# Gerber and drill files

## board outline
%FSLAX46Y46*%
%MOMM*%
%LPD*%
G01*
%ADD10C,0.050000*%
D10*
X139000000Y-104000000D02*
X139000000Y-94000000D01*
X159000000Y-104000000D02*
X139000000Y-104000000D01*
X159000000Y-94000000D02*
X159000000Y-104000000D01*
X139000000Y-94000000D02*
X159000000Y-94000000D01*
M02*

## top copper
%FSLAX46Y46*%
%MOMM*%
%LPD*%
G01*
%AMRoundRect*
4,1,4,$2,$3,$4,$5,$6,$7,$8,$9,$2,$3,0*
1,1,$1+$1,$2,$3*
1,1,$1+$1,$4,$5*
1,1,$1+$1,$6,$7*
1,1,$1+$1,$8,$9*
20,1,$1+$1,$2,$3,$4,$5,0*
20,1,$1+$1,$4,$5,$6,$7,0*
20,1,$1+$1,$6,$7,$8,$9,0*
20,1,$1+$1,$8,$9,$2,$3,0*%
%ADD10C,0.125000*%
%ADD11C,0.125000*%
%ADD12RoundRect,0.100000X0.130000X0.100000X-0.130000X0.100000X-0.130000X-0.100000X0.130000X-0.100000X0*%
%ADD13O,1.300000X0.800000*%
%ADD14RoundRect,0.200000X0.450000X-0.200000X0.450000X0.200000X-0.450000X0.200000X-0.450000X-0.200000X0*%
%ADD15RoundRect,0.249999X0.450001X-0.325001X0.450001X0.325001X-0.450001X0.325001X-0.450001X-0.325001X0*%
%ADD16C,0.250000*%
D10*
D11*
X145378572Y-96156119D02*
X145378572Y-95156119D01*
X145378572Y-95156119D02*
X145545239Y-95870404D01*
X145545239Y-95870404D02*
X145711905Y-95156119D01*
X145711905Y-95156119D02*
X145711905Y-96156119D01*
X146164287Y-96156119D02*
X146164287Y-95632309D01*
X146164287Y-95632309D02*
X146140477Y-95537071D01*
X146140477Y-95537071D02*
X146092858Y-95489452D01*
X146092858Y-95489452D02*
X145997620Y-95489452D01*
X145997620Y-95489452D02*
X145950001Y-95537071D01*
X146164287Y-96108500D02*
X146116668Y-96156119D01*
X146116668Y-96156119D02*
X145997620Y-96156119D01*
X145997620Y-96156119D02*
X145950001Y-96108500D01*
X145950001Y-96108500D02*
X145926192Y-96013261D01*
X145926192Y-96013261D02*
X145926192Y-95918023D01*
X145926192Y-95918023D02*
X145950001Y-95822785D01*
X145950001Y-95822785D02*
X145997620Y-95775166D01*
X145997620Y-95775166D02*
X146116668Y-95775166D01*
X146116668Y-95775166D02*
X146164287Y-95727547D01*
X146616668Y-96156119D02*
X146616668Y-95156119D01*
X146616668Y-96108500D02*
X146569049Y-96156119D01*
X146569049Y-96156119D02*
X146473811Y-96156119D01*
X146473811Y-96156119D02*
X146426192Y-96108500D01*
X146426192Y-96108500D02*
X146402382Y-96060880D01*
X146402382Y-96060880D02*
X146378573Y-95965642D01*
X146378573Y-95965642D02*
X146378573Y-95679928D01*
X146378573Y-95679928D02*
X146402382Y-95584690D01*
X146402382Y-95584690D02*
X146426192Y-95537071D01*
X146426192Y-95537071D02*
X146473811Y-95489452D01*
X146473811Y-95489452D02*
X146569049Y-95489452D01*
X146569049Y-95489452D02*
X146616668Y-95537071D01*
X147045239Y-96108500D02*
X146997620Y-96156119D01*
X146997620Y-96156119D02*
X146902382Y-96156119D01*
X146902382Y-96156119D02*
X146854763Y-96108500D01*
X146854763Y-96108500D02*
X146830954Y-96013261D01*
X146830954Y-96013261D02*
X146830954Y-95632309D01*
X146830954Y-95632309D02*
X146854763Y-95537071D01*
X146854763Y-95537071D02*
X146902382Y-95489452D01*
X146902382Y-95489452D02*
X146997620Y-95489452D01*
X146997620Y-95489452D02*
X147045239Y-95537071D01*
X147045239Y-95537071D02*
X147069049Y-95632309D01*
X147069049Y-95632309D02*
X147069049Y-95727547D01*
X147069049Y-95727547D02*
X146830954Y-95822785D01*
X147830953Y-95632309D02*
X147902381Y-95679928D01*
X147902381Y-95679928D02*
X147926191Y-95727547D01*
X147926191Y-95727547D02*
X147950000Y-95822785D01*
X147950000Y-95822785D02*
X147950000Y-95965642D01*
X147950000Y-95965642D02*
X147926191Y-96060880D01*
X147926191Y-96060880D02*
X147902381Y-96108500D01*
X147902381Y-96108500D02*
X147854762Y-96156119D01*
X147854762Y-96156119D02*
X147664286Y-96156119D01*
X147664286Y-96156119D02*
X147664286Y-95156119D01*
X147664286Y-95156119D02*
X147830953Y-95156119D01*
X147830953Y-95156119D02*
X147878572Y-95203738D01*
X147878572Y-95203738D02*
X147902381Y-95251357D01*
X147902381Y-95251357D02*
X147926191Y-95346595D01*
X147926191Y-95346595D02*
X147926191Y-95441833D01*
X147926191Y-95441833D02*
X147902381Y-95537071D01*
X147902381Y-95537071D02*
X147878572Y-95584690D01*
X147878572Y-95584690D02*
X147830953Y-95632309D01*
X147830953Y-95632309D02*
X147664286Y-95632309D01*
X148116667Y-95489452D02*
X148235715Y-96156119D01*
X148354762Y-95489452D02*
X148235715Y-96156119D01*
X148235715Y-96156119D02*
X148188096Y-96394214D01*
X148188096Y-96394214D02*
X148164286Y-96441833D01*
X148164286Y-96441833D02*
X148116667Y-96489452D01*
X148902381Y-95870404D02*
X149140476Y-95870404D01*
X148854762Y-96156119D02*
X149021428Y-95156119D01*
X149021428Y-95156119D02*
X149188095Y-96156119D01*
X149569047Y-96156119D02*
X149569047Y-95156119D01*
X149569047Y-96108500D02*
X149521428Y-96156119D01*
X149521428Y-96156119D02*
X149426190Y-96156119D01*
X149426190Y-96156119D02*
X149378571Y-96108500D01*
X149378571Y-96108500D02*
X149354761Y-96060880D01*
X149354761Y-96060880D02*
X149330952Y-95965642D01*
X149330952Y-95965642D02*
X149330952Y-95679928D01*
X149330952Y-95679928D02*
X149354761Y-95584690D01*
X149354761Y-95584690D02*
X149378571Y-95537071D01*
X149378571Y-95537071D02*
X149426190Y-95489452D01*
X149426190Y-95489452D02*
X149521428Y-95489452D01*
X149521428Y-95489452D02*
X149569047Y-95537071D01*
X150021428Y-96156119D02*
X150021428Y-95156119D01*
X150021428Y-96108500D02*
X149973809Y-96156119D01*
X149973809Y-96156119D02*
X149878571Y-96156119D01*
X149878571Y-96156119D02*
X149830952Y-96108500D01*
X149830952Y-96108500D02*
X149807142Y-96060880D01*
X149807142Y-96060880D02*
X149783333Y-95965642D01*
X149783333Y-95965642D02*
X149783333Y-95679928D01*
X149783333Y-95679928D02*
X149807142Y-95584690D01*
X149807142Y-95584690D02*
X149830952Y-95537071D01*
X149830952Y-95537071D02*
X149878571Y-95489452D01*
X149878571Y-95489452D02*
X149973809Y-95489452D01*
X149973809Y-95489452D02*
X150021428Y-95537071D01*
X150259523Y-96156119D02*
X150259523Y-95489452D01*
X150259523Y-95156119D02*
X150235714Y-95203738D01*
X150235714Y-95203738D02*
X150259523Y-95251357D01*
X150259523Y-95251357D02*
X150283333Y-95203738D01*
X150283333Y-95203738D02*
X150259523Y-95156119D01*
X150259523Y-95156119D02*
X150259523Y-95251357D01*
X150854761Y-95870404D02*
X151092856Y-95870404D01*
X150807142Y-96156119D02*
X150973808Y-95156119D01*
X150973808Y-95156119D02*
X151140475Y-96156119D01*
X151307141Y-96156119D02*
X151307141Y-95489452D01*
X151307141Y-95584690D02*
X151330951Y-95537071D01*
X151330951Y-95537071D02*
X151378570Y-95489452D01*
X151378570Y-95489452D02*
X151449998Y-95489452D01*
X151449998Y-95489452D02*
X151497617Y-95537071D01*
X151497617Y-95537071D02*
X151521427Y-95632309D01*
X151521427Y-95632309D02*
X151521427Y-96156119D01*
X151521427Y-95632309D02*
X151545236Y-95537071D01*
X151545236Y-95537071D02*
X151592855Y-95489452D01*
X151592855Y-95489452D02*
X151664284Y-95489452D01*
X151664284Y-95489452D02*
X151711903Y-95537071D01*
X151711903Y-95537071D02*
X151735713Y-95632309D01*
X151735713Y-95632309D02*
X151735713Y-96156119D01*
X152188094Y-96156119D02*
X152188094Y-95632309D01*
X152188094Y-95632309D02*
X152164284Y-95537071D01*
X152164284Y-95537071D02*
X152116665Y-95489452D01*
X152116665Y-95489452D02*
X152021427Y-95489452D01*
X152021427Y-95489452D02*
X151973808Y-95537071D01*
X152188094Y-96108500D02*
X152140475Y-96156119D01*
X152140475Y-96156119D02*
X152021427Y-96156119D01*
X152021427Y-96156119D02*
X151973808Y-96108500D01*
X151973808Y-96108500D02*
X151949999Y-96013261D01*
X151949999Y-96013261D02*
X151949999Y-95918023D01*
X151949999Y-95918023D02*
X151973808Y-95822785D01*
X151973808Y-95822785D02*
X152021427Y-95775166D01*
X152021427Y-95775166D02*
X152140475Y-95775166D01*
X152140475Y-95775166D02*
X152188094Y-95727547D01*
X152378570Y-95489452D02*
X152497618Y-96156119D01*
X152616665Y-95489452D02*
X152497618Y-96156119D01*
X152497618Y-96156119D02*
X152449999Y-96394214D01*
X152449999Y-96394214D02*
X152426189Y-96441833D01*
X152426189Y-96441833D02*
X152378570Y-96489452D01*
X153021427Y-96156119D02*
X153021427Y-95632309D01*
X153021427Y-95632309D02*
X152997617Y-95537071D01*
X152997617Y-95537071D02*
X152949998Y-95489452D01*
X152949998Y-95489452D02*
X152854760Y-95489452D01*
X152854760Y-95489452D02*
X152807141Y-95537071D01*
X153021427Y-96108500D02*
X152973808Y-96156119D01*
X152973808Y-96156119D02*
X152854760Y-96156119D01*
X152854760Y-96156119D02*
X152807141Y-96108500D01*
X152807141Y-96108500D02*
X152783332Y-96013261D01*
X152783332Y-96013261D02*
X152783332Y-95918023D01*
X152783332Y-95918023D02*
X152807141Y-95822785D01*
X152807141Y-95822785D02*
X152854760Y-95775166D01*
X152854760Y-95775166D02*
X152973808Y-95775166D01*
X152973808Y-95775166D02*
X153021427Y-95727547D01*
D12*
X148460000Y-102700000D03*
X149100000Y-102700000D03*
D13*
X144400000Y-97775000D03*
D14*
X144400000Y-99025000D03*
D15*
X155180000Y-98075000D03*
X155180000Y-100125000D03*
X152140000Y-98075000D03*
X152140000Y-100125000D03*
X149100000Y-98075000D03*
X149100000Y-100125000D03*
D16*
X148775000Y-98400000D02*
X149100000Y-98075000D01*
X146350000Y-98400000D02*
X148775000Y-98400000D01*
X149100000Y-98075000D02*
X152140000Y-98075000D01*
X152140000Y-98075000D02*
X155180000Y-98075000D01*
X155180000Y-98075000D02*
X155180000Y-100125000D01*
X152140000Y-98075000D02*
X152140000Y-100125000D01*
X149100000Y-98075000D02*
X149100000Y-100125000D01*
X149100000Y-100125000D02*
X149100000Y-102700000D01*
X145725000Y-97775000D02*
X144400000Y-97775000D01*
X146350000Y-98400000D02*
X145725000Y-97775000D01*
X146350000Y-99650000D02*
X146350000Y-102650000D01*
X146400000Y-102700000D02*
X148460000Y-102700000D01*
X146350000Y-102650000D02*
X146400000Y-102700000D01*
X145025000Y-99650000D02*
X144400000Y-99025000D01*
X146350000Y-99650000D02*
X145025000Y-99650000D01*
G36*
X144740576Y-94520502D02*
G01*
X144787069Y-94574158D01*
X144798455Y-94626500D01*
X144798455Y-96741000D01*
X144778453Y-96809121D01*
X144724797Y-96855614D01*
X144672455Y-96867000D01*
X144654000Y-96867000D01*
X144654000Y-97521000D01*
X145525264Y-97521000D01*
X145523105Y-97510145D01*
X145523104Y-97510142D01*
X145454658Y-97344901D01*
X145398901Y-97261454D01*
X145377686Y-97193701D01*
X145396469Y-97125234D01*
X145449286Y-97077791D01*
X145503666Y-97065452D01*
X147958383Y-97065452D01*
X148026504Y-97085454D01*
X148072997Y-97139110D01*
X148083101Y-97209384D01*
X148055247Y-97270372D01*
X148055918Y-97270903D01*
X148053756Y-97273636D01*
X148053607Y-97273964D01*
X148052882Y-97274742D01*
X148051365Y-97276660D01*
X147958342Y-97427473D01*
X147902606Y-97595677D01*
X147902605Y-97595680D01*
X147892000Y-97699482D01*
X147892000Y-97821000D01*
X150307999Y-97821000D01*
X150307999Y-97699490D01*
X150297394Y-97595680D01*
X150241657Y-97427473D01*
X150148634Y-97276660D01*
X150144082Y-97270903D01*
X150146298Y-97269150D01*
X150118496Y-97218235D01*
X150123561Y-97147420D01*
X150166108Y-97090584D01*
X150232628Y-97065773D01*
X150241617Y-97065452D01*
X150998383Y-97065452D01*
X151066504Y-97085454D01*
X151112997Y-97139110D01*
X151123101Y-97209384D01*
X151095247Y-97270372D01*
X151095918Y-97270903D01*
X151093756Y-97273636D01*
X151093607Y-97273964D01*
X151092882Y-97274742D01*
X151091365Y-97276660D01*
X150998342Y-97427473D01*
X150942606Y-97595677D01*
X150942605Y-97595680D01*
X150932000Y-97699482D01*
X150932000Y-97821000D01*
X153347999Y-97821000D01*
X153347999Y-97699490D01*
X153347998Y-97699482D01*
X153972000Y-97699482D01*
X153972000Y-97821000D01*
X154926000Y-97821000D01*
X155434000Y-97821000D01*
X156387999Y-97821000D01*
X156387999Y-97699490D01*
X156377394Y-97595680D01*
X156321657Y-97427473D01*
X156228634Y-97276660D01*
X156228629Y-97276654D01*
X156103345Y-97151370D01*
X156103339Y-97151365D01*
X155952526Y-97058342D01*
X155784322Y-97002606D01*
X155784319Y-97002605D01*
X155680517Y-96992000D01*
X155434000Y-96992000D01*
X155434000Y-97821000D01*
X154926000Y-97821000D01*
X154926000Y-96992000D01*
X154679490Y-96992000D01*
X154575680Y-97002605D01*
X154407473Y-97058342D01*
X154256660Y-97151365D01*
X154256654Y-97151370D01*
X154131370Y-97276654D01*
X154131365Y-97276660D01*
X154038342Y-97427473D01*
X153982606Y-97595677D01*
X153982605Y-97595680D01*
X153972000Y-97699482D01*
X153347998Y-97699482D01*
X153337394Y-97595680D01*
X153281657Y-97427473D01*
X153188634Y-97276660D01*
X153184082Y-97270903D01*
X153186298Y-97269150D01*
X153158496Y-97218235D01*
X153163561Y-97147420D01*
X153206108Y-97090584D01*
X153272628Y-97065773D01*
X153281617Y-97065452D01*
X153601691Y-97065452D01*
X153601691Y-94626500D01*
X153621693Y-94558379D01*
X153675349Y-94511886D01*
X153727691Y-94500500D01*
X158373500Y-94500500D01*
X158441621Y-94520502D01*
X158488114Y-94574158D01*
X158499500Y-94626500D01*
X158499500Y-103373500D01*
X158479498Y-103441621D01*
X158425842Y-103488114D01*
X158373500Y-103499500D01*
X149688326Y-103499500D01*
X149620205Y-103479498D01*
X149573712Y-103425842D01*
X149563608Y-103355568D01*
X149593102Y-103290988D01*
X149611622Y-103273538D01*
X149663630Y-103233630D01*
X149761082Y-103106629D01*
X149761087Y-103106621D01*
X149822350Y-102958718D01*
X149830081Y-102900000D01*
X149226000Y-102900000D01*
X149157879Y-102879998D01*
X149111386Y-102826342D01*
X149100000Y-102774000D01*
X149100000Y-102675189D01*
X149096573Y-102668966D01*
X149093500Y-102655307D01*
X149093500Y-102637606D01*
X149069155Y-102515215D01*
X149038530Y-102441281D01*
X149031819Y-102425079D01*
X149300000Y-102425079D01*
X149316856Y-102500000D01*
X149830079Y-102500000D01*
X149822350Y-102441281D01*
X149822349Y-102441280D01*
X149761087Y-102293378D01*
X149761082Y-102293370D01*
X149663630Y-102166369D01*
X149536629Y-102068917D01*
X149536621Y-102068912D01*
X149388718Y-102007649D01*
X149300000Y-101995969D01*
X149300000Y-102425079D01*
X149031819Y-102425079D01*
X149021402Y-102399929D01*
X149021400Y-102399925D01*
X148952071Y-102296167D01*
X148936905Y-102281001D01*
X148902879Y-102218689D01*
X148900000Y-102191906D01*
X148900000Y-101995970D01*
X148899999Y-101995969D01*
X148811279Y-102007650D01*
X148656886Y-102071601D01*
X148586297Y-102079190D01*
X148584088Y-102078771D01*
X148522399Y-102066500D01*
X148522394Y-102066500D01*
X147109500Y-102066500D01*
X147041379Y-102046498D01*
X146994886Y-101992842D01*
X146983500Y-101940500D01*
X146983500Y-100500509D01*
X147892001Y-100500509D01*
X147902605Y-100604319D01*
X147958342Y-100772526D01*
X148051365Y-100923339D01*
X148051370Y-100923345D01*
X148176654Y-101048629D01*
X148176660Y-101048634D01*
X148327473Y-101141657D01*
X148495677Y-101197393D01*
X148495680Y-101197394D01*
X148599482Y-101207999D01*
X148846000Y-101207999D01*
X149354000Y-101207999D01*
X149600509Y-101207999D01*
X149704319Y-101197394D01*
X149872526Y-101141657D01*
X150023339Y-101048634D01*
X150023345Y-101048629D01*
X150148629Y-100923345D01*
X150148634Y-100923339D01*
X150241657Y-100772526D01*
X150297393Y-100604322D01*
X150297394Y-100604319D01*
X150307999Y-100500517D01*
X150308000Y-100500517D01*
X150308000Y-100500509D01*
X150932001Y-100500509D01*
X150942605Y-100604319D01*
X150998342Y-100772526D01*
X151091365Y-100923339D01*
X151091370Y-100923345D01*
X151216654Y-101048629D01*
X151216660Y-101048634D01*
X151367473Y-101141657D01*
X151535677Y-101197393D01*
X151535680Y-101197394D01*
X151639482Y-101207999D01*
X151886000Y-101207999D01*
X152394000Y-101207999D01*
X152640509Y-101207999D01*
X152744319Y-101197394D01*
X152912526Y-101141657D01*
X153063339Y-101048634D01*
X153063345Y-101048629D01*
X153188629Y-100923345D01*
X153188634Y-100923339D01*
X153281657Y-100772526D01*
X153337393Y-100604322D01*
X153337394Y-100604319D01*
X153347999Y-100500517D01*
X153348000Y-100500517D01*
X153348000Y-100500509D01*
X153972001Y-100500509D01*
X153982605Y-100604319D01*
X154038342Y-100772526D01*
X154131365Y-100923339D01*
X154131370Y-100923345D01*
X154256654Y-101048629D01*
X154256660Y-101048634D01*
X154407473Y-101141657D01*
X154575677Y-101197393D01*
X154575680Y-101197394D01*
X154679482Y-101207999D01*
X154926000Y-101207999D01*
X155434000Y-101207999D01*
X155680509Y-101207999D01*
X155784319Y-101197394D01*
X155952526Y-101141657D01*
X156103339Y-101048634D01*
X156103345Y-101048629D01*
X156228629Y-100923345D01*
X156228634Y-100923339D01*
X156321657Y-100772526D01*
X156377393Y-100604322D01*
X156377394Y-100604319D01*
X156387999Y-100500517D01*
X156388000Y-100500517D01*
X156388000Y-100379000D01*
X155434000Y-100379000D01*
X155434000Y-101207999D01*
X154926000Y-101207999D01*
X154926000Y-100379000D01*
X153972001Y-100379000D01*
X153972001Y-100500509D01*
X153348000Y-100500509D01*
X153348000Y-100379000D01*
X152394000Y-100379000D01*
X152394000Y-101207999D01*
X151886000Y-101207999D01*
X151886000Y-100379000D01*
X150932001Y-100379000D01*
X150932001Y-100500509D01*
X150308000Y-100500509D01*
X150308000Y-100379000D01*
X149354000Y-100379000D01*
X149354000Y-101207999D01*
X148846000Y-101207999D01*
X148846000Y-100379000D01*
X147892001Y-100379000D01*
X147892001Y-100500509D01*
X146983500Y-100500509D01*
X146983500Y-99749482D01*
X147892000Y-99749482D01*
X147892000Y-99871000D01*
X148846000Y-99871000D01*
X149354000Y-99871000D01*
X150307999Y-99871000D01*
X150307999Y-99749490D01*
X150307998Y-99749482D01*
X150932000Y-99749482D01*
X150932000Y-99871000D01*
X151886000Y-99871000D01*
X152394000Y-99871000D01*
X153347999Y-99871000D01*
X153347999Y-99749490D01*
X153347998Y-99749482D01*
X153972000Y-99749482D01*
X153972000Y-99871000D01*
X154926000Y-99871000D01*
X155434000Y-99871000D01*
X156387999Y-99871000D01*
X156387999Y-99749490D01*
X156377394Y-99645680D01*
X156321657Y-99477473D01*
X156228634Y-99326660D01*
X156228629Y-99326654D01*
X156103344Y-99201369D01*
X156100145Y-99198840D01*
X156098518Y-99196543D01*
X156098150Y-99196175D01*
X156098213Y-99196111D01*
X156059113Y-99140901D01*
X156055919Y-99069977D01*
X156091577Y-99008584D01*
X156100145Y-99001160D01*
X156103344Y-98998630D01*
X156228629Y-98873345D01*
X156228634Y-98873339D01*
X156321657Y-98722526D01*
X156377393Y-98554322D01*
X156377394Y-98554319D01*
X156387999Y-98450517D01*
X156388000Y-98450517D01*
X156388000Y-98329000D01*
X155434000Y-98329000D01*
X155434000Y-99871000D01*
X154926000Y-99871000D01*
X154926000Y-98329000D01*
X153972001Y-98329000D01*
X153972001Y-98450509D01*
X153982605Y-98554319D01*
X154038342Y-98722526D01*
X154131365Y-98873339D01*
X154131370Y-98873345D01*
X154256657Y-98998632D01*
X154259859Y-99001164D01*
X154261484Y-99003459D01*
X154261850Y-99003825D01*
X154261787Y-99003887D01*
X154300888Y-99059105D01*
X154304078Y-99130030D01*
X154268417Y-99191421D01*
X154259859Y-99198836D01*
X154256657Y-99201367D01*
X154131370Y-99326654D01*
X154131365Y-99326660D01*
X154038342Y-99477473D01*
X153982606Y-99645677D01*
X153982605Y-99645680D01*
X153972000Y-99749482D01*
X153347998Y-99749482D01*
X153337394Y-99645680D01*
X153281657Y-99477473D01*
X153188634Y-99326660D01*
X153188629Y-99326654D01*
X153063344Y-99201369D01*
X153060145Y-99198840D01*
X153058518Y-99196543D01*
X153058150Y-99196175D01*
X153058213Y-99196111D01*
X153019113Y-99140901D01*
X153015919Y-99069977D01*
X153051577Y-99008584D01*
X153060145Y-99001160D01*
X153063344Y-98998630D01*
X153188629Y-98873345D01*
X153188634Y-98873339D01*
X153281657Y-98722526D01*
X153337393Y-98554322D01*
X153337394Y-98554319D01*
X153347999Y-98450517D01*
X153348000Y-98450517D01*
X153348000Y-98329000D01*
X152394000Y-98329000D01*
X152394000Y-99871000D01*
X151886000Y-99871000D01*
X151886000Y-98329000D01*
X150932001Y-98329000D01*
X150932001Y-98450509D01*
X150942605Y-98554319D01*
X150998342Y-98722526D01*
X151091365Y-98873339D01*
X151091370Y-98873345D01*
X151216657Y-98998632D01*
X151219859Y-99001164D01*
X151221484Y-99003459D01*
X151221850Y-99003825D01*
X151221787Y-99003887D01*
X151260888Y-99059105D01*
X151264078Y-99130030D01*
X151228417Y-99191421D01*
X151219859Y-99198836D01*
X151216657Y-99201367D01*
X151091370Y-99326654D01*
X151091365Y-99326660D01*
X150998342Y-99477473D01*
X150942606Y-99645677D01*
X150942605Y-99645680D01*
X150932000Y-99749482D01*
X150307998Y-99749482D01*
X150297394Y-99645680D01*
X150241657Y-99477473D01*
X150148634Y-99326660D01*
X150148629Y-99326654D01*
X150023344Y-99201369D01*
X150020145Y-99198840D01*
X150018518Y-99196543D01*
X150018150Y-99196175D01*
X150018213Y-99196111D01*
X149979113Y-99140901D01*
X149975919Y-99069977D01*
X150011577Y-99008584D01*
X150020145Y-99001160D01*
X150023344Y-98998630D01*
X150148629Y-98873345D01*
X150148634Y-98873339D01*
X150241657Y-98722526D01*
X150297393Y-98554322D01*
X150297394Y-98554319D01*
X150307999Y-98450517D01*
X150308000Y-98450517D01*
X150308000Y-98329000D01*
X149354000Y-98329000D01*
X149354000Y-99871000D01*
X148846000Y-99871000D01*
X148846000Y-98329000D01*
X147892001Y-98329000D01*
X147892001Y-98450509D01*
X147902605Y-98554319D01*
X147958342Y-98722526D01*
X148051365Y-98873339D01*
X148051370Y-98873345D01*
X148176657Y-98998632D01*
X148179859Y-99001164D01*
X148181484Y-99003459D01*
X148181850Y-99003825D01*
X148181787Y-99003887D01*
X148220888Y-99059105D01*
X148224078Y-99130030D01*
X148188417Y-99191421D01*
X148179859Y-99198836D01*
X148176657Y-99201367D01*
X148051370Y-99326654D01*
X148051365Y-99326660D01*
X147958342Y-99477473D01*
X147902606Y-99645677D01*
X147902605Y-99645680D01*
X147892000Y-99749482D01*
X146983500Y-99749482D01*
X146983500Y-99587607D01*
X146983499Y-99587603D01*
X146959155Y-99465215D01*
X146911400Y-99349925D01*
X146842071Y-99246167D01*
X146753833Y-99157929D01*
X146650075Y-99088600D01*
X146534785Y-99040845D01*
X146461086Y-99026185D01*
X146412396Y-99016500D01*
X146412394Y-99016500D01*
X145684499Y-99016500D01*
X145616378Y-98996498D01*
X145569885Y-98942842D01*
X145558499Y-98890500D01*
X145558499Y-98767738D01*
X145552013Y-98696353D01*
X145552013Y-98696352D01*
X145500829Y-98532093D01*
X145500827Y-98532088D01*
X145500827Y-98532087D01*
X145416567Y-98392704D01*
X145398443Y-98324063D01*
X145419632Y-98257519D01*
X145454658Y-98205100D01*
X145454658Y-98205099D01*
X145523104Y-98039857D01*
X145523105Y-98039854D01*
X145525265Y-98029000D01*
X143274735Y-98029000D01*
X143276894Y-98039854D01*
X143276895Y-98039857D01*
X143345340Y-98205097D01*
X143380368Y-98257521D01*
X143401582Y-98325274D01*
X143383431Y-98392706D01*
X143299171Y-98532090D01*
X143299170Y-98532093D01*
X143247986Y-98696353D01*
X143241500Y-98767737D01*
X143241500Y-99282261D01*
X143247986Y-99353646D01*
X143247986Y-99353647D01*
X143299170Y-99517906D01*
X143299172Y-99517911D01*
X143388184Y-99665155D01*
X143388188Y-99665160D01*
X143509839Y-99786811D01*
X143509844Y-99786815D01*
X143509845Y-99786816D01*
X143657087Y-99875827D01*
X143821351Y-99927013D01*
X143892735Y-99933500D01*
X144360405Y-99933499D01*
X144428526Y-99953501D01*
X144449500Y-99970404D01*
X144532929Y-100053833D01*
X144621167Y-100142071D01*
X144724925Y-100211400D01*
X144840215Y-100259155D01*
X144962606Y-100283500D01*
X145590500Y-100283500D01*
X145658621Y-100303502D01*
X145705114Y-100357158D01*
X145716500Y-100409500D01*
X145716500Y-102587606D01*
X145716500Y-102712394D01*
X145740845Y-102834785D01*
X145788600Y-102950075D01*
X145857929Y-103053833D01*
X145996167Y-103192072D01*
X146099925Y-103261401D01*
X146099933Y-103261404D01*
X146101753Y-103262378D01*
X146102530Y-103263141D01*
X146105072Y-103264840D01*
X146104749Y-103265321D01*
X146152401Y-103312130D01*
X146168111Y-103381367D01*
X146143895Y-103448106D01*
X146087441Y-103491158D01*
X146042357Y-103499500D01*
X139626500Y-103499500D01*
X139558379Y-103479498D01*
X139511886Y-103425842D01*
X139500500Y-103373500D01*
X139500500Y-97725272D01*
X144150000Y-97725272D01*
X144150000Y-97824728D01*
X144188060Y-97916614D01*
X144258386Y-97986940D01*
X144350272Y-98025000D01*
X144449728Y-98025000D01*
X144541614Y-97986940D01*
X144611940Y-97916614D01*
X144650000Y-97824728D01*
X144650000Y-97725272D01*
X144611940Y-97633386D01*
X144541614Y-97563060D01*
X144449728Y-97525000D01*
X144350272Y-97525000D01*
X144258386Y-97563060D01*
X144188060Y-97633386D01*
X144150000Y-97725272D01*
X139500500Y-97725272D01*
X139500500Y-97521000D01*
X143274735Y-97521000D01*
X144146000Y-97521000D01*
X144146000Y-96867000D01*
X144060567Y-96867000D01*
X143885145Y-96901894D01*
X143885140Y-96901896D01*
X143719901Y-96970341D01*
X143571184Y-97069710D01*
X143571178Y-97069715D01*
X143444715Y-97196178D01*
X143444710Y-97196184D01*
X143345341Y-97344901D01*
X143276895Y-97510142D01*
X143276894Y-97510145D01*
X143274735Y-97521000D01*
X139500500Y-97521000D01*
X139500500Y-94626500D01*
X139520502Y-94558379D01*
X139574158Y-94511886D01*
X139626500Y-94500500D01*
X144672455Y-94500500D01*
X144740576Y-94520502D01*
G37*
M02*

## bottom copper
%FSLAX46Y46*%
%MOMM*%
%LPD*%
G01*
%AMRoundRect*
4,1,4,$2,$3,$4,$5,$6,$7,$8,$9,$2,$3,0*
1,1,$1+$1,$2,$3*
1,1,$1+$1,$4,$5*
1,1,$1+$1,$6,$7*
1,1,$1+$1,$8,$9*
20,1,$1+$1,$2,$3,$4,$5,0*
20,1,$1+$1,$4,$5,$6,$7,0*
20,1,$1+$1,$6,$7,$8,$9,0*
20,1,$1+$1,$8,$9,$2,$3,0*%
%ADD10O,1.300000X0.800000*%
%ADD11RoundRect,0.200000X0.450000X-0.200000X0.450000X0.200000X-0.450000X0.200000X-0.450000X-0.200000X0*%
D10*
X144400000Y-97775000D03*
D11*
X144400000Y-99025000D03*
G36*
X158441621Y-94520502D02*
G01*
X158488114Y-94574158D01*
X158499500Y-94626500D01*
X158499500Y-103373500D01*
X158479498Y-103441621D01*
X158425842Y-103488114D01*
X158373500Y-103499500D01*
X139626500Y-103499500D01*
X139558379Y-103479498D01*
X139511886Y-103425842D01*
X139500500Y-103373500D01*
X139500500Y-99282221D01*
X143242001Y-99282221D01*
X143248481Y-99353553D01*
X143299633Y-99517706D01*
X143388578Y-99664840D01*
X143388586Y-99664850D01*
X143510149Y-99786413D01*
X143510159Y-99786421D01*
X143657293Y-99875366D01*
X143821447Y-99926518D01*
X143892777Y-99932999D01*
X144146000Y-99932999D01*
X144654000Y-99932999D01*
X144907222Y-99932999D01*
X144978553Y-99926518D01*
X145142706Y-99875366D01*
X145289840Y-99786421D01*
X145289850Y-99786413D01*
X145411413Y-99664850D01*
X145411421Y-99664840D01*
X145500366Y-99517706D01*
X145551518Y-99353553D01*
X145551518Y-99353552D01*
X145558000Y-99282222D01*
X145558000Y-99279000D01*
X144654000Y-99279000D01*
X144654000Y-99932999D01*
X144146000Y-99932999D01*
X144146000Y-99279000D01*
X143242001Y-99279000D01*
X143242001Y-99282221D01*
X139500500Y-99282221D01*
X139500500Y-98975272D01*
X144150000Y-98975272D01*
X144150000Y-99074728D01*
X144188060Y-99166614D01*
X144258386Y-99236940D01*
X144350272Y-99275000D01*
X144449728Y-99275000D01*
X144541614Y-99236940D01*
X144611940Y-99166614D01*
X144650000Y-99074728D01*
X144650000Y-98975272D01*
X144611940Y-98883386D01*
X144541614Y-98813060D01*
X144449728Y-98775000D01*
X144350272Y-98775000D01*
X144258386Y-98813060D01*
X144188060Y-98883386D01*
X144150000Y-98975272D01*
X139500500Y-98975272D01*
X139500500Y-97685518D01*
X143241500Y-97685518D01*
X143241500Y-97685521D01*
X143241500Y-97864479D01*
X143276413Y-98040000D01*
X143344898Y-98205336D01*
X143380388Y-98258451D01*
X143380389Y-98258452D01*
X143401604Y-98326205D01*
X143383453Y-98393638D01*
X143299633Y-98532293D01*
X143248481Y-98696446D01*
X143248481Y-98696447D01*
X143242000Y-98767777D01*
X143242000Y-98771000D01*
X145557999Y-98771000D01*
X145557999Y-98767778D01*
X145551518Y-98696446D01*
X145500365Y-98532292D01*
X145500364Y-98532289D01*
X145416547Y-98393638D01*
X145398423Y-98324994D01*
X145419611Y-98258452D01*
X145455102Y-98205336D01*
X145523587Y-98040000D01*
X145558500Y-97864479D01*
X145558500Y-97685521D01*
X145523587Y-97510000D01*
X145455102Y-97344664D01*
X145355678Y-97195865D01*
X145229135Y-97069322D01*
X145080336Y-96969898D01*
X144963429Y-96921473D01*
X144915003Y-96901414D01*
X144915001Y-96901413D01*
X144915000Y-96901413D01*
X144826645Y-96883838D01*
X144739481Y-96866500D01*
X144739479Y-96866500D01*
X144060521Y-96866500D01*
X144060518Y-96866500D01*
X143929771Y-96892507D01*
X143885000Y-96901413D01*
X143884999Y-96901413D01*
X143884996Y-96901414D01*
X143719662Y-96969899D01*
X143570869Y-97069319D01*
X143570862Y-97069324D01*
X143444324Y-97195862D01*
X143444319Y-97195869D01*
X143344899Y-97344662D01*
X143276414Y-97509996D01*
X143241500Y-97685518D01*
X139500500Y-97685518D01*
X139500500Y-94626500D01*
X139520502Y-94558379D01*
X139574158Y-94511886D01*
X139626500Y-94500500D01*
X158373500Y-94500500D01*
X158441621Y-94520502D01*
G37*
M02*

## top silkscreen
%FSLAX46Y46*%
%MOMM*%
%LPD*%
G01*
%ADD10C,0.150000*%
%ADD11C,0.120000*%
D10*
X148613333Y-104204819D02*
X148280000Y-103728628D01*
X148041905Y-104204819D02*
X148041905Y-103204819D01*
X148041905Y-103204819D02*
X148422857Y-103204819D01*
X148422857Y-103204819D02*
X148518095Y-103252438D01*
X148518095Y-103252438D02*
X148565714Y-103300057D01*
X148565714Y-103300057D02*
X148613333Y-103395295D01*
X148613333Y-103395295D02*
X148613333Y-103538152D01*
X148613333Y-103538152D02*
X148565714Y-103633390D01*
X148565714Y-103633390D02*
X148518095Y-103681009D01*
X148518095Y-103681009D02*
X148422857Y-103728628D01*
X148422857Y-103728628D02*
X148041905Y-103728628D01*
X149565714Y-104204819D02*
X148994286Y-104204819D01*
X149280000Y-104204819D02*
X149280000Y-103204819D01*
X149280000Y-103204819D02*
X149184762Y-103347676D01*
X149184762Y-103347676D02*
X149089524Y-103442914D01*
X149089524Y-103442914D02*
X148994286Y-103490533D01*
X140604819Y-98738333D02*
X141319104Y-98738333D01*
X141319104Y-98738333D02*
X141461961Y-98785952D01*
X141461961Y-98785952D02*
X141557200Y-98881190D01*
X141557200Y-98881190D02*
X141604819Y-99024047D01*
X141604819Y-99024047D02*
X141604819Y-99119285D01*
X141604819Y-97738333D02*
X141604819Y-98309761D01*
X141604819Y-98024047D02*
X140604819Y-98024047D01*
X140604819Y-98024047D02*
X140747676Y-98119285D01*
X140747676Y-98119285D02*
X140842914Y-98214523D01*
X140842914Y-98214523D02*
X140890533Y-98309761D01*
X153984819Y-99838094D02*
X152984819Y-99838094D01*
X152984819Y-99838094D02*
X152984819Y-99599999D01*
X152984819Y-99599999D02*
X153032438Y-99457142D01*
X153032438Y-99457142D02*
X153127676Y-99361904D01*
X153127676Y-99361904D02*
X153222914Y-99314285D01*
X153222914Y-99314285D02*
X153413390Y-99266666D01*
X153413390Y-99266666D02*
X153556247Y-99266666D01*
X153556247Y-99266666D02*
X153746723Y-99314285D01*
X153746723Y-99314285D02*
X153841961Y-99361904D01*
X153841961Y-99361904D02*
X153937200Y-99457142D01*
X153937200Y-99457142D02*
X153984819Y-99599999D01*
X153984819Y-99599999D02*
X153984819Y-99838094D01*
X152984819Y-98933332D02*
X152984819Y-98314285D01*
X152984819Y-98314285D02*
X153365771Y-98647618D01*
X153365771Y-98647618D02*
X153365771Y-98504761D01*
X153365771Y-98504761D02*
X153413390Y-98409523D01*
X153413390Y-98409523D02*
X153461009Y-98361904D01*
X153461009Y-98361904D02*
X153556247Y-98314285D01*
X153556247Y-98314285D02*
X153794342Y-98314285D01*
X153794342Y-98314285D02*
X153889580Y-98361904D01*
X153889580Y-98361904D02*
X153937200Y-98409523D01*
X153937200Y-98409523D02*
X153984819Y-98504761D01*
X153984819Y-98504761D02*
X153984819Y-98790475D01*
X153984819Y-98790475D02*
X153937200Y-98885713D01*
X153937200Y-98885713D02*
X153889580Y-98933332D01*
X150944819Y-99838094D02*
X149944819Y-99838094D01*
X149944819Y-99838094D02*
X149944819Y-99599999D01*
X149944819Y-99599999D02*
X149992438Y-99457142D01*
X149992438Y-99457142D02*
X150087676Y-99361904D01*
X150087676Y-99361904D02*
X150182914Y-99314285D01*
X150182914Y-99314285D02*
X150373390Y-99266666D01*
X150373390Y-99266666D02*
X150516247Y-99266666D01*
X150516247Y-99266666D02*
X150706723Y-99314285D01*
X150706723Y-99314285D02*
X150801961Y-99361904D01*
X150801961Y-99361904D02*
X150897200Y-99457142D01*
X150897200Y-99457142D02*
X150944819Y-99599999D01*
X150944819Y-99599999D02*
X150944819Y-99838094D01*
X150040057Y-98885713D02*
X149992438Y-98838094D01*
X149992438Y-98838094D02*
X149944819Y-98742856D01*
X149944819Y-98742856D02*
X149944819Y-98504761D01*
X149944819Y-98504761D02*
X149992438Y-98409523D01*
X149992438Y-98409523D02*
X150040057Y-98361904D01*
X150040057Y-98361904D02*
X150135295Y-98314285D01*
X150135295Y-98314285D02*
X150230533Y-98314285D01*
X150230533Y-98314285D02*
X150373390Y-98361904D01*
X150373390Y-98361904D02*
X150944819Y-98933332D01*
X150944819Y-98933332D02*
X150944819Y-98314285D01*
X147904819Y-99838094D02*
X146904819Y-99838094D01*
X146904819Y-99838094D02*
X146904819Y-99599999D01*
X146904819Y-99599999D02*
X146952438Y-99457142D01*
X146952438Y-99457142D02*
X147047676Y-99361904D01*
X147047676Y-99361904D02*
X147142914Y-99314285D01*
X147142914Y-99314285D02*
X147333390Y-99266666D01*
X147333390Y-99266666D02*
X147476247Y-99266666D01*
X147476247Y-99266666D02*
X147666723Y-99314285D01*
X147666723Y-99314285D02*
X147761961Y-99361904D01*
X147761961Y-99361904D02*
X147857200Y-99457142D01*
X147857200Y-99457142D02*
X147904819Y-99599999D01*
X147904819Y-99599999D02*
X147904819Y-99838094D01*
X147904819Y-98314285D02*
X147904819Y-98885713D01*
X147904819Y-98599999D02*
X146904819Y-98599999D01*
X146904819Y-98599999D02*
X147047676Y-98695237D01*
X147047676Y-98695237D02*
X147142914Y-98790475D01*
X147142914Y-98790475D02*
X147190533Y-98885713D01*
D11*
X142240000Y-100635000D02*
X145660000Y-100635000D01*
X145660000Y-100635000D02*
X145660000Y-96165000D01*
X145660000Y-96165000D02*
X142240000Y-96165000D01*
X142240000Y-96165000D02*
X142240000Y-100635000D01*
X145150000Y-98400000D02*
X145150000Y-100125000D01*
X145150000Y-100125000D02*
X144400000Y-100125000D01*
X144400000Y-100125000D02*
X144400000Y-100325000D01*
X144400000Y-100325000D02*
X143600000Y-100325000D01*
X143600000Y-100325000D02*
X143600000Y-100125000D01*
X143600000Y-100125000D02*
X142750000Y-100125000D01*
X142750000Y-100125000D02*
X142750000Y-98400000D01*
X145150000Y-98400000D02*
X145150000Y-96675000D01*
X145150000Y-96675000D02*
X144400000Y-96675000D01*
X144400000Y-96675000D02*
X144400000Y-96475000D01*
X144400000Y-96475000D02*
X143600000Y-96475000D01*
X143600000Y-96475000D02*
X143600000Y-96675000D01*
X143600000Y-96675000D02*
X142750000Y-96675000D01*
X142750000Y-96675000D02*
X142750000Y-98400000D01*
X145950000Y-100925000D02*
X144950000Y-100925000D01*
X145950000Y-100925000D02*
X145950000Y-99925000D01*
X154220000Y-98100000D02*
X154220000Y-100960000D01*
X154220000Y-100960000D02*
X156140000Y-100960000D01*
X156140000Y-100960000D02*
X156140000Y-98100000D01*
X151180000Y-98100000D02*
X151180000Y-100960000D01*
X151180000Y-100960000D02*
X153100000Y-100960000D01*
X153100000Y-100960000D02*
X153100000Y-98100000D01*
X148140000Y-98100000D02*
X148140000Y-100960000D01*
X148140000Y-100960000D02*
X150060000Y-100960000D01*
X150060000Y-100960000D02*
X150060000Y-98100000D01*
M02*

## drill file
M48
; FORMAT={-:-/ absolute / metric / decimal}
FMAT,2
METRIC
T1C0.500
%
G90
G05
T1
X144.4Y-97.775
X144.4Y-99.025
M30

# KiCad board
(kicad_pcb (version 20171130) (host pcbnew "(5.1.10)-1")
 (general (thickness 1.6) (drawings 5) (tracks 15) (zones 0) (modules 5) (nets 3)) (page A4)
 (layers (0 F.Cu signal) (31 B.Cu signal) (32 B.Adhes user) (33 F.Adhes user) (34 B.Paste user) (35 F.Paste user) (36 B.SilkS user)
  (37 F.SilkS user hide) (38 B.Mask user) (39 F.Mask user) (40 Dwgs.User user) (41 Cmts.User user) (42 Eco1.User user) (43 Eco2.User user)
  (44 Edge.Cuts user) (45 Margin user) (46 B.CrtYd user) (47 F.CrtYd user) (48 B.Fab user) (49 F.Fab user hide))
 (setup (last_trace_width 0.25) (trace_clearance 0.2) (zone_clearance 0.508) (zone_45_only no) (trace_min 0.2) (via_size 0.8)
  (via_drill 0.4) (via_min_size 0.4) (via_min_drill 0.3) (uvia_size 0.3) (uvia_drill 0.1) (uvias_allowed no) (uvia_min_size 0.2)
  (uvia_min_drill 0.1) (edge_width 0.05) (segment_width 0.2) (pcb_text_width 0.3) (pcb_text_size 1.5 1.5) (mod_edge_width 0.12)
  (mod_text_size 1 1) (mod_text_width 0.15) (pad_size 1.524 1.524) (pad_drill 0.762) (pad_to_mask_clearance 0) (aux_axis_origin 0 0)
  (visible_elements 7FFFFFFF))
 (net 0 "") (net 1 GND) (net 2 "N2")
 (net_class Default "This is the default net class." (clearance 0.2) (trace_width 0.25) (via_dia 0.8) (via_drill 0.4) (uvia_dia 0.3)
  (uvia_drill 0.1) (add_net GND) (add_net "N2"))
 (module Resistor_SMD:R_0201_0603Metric (layer F.Cu) (at 148.78 102.7 180) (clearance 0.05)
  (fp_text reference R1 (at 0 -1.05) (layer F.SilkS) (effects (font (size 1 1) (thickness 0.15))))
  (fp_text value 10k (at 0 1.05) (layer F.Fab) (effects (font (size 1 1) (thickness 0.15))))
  (pad 2 smd roundrect (at 0.32 0 180) (size 0.46 0.4) (layers F.Cu F.Mask) (roundrect_rratio 0.25) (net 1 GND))
  (pad 1 smd roundrect (at -0.32 0 180) (size 0.46 0.4) (layers F.Cu F.Mask) (roundrect_rratio 0.25) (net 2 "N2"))
  (pad "" smd roundrect (at 0.345 0 180) (size 0.318 0.36) (layers F.Paste) (roundrect_rratio 0.25))
  (pad "" smd roundrect (at -0.345 0 180) (size 0.318 0.36) (layers F.Paste) (roundrect_rratio 0.25)))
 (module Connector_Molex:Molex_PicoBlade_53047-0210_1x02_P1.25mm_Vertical (layer F.Cu) (at 144.4 99.025 90)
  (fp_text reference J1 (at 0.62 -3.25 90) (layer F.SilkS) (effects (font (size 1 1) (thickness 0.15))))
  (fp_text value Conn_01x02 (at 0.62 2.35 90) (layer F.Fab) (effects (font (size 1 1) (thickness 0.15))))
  (fp_line (start -1.61 -2.16) (end -1.61 1.26) (layer F.SilkS) (width 0.12))
  (fp_line (start -1.61 1.26) (end 2.86 1.26) (layer F.SilkS) (width 0.12))
  (fp_line (start 2.86 1.26) (end 2.86 -2.16) (layer F.SilkS) (width 0.12))
  (fp_line (start 2.86 -2.16) (end -1.61 -2.16) (layer F.SilkS) (width 0.12))
  (fp_line (start 0.625 0.75) (end -1.1 0.75) (layer F.SilkS) (width 0.12))
  (fp_line (start -1.1 0.75) (end -1.1 0) (layer F.SilkS) (width 0.12))
  (fp_line (start -1.1 0) (end -1.3 0) (layer F.SilkS) (width 0.12))
  (fp_line (start -1.3 0) (end -1.3 -0.8) (layer F.SilkS) (width 0.12))
  (fp_line (start -1.3 -0.8) (end -1.1 -0.8) (layer F.SilkS) (width 0.12))
  (fp_line (start -1.1 -0.8) (end -1.1 -1.65) (layer F.SilkS) (width 0.12))
  (fp_line (start -1.1 -1.65) (end 0.625 -1.65) (layer F.SilkS) (width 0.12))
  (fp_line (start 0.625 0.75) (end 2.35 0.75) (layer F.SilkS) (width 0.12))
  (fp_line (start 2.35 0.75) (end 2.35 0) (layer F.SilkS) (width 0.12))
  (fp_line (start 2.35 0) (end 2.55 0) (layer F.SilkS) (width 0.12))
  (fp_line (start 2.55 0) (end 2.55 -0.8) (layer F.SilkS) (width 0.12))
  (fp_line (start 2.55 -0.8) (end 2.35 -0.8) (layer F.SilkS) (width 0.12))
  (fp_line (start 2.35 -0.8) (end 2.35 -1.65) (layer F.SilkS) (width 0.12))
  (fp_line (start 2.35 -1.65) (end 0.625 -1.65) (layer F.SilkS) (width 0.12))
  (fp_line (start -1.9 1.55) (end -1.9 0.55) (layer F.SilkS) (width 0.12))
  (fp_line (start -1.9 1.55) (end -0.9 1.55) (layer F.SilkS) (width 0.12))
  (pad 2 thru_hole oval (at 1.25 0 90) (size 0.8 1.3) (drill 0.5) (layers *.Cu *.Mask) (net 2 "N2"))
  (pad 1 thru_hole roundrect (at 0 0 90) (size 0.8 1.3) (drill 0.5) (layers *.Cu *.Mask) (roundrect_rratio 0.25) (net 1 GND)))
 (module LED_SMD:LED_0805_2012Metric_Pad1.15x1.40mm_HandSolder (layer F.Cu) (at 155.18 99.1 90)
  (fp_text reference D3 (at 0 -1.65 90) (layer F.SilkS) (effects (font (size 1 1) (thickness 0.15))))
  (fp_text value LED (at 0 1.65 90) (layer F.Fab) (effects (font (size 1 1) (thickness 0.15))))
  (fp_line (start 1 -0.96) (end -1.86 -0.96) (layer F.SilkS) (width 0.12))
  (fp_line (start -1.86 -0.96) (end -1.86 0.96) (layer F.SilkS) (width 0.12))
  (fp_line (start -1.86 0.96) (end 1 0.96) (layer F.SilkS) (width 0.12))
  (pad 2 smd roundrect (at 1.025 0 90) (size 1.15 1.4) (layers F.Cu F.Paste F.Mask) (roundrect_rratio 0.2173904347826087) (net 2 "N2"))
  (pad 1 smd roundrect (at -1.025 0 90) (size 1.15 1.4) (layers F.Cu F.Paste F.Mask) (roundrect_rratio 0.2173904347826087) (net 2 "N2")))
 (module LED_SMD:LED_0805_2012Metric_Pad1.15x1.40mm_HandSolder (layer F.Cu) (at 152.14 99.1 90)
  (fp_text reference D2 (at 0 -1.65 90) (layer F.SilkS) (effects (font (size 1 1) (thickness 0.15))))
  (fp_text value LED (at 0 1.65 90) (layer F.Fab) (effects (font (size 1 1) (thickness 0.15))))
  (fp_line (start 1 -0.96) (end -1.86 -0.96) (layer F.SilkS) (width 0.12))
  (fp_line (start -1.86 -0.96) (end -1.86 0.96) (layer F.SilkS) (width 0.12))
  (fp_line (start -1.86 0.96) (end 1 0.96) (layer F.SilkS) (width 0.12))
  (pad 2 smd roundrect (at 1.025 0 90) (size 1.15 1.4) (layers F.Cu F.Paste F.Mask) (roundrect_rratio 0.2173904347826087) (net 2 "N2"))
  (pad 1 smd roundrect (at -1.025 0 90) (size 1.15 1.4) (layers F.Cu F.Paste F.Mask) (roundrect_rratio 0.2173904347826087) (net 2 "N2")))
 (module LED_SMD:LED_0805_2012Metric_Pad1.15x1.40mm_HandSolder (layer F.Cu) (at 149.1 99.1 90)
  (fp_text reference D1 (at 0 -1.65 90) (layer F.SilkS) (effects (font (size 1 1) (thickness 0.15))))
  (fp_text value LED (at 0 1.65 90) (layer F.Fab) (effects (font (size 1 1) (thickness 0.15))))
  (fp_line (start 1 -0.96) (end -1.86 -0.96) (layer F.SilkS) (width 0.12))
  (fp_line (start -1.86 -0.96) (end -1.86 0.96) (layer F.SilkS) (width 0.12))
  (fp_line (start -1.86 0.96) (end 1 0.96) (layer F.SilkS) (width 0.12))
  (pad 2 smd roundrect (at 1.025 0 90) (size 1.15 1.4) (layers F.Cu F.Paste F.Mask) (roundrect_rratio 0.2173904347826087) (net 2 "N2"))
  (pad 1 smd roundrect (at -1.025 0 90) (size 1.15 1.4) (layers F.Cu F.Paste F.Mask) (roundrect_rratio 0.2173904347826087) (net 2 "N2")))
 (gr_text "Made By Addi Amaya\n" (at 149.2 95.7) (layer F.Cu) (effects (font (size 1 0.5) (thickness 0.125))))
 (gr_line (start 139 104) (end 139 94) (layer Edge.Cuts) (width 0.05))
 (gr_line (start 159 104) (end 139 104) (layer Edge.Cuts) (width 0.05))
 (gr_line (start 159 94) (end 159 104) (layer Edge.Cuts) (width 0.05))
 (gr_line (start 139 94) (end 159 94) (layer Edge.Cuts) (width 0.05))
 (segment (start 148.775 98.4) (end 149.1 98.075) (width 0.25) (layer F.Cu) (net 2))
 (segment (start 146.35 98.4) (end 148.775 98.4) (width 0.25) (layer F.Cu) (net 2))
 (segment (start 149.1 98.075) (end 152.14 98.075) (width 0.25) (layer F.Cu) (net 2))
 (segment (start 152.14 98.075) (end 155.18 98.075) (width 0.25) (layer F.Cu) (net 2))
 (segment (start 155.18 98.075) (end 155.18 100.125) (width 0.25) (layer F.Cu) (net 2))
 (segment (start 152.14 98.075) (end 152.14 100.125) (width 0.25) (layer F.Cu) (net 2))
 (segment (start 149.1 98.075) (end 149.1 100.125) (width 0.25) (layer F.Cu) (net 2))
 (segment (start 149.1 100.125) (end 149.1 102.7) (width 0.25) (layer F.Cu) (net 2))
 (segment (start 145.725 97.775) (end 144.4 97.775) (width 0.25) (layer F.Cu) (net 2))
 (segment (start 146.35 98.4) (end 145.725 97.775) (width 0.25) (layer F.Cu) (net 2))
 (segment (start 146.35 99.65) (end 146.35 102.65) (width 0.25) (layer F.Cu) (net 1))
 (segment (start 146.4 102.7) (end 148.46 102.7) (width 0.25) (layer F.Cu) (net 1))
 (segment (start 146.35 102.65) (end 146.4 102.7) (width 0.25) (layer F.Cu) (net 1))
 (segment (start 145.025 99.65) (end 144.4 99.025) (width 0.25) (layer F.Cu) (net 1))
 (segment (start 146.35 99.65) (end 145.025 99.65) (width 0.25) (layer F.Cu) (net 1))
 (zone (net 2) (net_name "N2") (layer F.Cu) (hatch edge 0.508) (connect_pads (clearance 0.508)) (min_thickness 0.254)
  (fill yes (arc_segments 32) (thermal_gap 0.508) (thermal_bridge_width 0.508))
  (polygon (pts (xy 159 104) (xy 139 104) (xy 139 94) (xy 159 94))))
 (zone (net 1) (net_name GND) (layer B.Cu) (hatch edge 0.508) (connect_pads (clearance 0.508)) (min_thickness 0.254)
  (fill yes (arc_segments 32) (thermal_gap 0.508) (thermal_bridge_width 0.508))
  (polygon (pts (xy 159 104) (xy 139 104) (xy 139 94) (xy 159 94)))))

